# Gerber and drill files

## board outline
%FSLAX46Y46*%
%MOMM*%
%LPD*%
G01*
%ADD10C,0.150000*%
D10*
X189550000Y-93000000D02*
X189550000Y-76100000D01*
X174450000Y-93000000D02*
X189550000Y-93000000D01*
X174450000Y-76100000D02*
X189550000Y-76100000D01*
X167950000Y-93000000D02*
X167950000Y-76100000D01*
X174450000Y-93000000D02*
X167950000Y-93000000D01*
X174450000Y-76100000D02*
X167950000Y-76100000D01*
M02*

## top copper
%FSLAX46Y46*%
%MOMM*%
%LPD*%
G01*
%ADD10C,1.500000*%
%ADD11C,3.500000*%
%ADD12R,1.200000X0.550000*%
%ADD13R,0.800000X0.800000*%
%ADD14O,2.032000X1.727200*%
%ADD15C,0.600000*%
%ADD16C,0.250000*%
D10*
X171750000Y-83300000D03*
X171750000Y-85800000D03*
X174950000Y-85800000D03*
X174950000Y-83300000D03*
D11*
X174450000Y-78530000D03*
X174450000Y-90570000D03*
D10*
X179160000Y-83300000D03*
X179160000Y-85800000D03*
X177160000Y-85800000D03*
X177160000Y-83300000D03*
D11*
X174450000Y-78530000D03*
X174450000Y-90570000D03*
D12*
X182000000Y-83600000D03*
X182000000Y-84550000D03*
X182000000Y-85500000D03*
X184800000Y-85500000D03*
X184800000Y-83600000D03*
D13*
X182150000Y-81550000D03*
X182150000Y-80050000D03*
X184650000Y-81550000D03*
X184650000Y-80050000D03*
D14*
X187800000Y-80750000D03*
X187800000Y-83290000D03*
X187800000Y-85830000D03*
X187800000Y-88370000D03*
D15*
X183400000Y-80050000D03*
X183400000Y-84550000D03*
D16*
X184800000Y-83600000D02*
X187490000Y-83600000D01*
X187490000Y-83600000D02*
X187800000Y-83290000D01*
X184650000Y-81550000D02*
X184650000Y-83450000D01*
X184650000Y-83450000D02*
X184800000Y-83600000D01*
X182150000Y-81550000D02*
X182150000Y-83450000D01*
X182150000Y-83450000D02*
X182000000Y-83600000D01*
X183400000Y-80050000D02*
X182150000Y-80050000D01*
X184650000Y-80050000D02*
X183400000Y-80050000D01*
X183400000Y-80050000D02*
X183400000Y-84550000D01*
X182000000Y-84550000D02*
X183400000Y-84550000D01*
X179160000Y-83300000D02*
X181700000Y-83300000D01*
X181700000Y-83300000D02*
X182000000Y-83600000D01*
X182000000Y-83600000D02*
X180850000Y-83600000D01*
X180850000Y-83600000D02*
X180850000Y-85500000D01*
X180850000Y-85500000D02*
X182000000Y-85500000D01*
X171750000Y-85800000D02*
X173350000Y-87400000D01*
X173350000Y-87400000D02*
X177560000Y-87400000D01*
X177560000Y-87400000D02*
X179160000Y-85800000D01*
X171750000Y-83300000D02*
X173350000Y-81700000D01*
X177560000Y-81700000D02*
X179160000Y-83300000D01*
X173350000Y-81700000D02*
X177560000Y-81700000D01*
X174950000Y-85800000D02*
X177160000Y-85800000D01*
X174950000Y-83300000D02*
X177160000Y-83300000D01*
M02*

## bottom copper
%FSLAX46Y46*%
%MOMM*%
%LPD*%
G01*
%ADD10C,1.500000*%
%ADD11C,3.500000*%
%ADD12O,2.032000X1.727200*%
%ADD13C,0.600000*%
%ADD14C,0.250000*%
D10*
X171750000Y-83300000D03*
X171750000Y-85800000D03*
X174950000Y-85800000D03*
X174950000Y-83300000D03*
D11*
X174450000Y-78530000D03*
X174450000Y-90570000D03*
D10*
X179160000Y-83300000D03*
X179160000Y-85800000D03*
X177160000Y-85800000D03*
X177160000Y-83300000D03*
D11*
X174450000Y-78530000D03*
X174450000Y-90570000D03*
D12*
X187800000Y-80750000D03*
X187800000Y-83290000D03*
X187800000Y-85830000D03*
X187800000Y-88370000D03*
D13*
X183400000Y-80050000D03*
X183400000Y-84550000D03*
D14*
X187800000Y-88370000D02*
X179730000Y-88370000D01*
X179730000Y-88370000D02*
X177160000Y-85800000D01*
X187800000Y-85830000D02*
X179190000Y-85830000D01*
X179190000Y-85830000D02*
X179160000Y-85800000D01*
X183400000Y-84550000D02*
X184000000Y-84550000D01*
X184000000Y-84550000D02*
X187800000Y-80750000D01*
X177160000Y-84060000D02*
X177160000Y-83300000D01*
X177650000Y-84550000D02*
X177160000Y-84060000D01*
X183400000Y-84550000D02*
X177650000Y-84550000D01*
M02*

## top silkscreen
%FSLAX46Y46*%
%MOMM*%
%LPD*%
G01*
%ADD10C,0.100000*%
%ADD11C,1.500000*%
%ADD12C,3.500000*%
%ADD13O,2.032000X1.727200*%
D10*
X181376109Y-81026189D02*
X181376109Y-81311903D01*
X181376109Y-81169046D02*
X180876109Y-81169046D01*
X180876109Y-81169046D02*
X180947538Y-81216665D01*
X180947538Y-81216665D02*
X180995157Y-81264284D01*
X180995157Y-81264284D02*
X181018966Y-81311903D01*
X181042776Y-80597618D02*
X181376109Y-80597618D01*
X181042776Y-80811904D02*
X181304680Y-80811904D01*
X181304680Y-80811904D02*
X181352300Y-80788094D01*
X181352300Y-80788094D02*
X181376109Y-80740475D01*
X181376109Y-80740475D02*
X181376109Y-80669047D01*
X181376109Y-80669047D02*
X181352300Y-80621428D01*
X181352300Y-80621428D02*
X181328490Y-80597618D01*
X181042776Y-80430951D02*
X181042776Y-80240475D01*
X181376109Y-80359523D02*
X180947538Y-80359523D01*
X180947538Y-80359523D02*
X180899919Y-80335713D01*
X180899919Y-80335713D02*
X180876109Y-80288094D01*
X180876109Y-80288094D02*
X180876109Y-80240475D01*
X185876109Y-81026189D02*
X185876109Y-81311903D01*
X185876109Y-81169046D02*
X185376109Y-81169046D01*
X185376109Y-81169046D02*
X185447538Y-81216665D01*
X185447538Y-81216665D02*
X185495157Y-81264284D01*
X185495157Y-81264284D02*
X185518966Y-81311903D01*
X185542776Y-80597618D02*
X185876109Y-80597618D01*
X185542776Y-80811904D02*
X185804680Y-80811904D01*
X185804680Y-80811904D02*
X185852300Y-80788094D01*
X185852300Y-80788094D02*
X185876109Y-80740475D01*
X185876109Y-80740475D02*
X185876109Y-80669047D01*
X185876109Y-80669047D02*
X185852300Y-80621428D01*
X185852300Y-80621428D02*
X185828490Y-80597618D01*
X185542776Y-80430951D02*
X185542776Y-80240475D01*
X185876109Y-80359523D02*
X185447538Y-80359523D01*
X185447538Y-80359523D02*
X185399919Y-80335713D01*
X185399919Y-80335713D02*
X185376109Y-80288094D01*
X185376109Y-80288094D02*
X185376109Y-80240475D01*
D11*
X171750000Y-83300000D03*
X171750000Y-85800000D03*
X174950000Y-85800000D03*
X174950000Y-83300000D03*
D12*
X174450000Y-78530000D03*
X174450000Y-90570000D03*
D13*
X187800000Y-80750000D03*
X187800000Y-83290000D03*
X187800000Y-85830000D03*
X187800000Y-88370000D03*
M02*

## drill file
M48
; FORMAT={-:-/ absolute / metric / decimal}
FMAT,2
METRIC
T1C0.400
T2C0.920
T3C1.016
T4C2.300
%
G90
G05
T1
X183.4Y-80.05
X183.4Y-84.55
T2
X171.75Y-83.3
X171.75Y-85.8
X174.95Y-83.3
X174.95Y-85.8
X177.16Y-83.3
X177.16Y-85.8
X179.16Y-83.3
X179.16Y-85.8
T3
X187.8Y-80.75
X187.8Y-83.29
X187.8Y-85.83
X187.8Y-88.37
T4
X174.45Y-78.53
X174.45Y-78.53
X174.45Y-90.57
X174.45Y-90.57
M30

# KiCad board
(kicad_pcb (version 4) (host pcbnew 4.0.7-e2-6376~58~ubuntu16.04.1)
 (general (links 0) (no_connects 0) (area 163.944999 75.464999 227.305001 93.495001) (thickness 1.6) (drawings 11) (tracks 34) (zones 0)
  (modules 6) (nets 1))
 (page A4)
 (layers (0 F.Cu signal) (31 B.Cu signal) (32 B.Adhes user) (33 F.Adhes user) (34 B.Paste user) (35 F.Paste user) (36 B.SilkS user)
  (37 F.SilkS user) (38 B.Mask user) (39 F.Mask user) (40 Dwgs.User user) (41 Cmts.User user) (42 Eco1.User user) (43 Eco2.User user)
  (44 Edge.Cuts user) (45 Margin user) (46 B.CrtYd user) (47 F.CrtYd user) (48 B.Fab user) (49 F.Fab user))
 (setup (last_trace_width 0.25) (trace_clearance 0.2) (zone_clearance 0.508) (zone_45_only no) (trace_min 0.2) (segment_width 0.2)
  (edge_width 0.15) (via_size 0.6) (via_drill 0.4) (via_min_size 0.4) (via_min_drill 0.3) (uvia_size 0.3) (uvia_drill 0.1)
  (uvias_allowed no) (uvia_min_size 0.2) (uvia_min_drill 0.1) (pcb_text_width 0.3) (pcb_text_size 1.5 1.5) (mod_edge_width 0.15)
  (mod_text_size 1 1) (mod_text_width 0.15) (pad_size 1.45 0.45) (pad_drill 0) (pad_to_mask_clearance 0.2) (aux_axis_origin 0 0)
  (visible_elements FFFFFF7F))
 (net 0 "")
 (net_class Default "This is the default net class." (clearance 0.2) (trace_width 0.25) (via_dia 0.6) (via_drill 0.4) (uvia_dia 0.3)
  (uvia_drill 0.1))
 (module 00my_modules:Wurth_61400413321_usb (layer F.Cu) (at 174.45 84.55 90)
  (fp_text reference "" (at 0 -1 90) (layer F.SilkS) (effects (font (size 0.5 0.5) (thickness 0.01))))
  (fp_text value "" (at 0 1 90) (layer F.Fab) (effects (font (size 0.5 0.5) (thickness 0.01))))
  (pad V thru_hole circle (at 1.25 -2.7 90) (size 1.5 1.5) (drill 0.92) (layers *.Cu *.Mask F.SilkS))
  (pad - thru_hole circle (at -1.25 -2.7 90) (size 1.5 1.5) (drill 0.92) (layers *.Cu *.Mask F.SilkS))
  (pad + thru_hole circle (at -1.25 0.5 90) (size 1.5 1.5) (drill 0.92) (layers *.Cu *.Mask F.SilkS))
  (pad G thru_hole circle (at 1.25 0.5 90) (size 1.5 1.5) (drill 0.92) (layers *.Cu *.Mask F.SilkS))
  (pad X thru_hole circle (at 6.02 0 90) (size 3.5 3.5) (drill 2.3) (layers *.Cu *.Mask F.SilkS))
  (pad X thru_hole circle (at -6.02 0 90) (size 3.5 3.5) (drill 2.3) (layers *.Cu *.Mask F.SilkS)))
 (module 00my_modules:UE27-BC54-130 (layer B.Cu) (at 174.45 84.55 90)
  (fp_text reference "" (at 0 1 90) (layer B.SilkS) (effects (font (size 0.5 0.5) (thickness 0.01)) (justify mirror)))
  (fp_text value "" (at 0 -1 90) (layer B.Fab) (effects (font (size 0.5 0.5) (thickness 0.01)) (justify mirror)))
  (pad V thru_hole circle (at 1.25 4.71 90) (size 1.5 1.5) (drill 0.92) (layers *.Cu *.Mask B.SilkS))
  (pad - thru_hole circle (at -1.25 4.71 90) (size 1.5 1.5) (drill 0.92) (layers *.Cu *.Mask B.SilkS))
  (pad + thru_hole circle (at -1.25 2.71 90) (size 1.5 1.5) (drill 0.92) (layers *.Cu *.Mask B.SilkS))
  (pad G thru_hole circle (at 1.25 2.71 90) (size 1.5 1.5) (drill 0.92) (layers *.Cu *.Mask B.SilkS))
  (pad X thru_hole circle (at 6.02 0 90) (size 3.5 3.5) (drill 2.3) (layers *.Cu *.Mask B.SilkS))
  (pad X thru_hole circle (at -6.02 0 90) (size 3.5 3.5) (drill 2.3) (layers *.Cu *.Mask B.SilkS)))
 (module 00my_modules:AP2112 (layer F.Cu) (at 183.4 84.55)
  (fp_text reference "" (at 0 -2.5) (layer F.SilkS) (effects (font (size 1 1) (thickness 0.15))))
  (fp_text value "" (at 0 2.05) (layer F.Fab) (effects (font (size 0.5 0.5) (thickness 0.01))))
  (pad VIN smd rect (at -1.4 -0.95) (size 1.2 0.55) (layers F.Cu F.Paste F.Mask))
  (pad GND smd rect (at -1.4 0) (size 1.2 0.55) (layers F.Cu F.Paste F.Mask))
  (pad EN smd rect (at -1.4 0.95) (size 1.2 0.55) (layers F.Cu F.Paste F.Mask))
  (pad NC smd rect (at 1.4 0.95) (size 1.2 0.55) (layers F.Cu F.Paste F.Mask))
  (pad VOUT smd rect (at 1.4 -0.95) (size 1.2 0.55) (layers F.Cu F.Paste F.Mask)))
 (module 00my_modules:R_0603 (layer F.Cu) (at 182.15 80.8 90)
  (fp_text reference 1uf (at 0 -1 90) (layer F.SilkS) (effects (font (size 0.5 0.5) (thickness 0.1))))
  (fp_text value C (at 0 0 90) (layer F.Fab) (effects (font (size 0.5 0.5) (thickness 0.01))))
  (pad 1 smd rect (at -0.75 0 90) (size 0.8 0.8) (layers F.Cu F.Paste F.Mask))
  (pad 2 smd rect (at 0.75 0 90) (size 0.8 0.8) (layers F.Cu F.Paste F.Mask)))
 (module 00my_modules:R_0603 (layer F.Cu) (at 184.65 80.8 90)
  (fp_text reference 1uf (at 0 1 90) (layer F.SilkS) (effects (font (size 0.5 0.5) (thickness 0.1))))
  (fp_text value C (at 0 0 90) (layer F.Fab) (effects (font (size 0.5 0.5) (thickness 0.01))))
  (pad 1 smd rect (at -0.75 0 90) (size 0.8 0.8) (layers F.Cu F.Paste F.Mask))
  (pad 2 smd rect (at 0.75 0 90) (size 0.8 0.8) (layers F.Cu F.Paste F.Mask)))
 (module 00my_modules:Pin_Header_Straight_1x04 (layer F.Cu) (at 187.8 80.75)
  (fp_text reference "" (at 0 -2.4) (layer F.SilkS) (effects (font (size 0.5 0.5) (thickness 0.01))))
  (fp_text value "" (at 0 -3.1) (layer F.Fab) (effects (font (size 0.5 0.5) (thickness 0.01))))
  (pad 1 thru_hole oval (at 0 0) (size 2.032 1.7272) (drill 1.016) (layers *.Cu *.Mask F.SilkS))
  (pad 2 thru_hole oval (at 0 2.54) (size 2.032 1.7272) (drill 1.016) (layers *.Cu *.Mask F.SilkS))
  (pad 3 thru_hole oval (at 0 5.08) (size 2.032 1.7272) (drill 1.016) (layers *.Cu *.Mask F.SilkS))
  (pad 4 thru_hole oval (at 0 7.62) (size 2.032 1.7272) (drill 1.016) (layers *.Cu *.Mask F.SilkS)))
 (gr_line (start 189.55 93) (end 189.55 76.1) (angle 90) (layer Edge.Cuts) (width 0.15))
 (gr_line (start 174.45 93) (end 189.55 93) (angle 90) (layer Edge.Cuts) (width 0.15))
 (gr_line (start 174.45 76.1) (end 189.55 76.1) (angle 90) (layer Edge.Cuts) (width 0.15))
 (gr_line (start 167.95 93) (end 167.95 76.1) (angle 90) (layer Edge.Cuts) (width 0.15))
 (gr_line (start 174.45 93) (end 167.95 93) (angle 90) (layer Edge.Cuts) (width 0.15))
 (gr_line (start 174.45 76.1) (end 167.95 76.1) (angle 90) (layer Edge.Cuts) (width 0.15))
 (segment (start 187.8 88.37) (end 179.73 88.37) (width 0.25) (layer B.Cu) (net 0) (status 400000))
 (segment (start 179.73 88.37) (end 177.16 85.8) (width 0.25) (layer B.Cu) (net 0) (status 800000))
 (segment (start 187.8 85.83) (end 179.19 85.83) (width 0.25) (layer B.Cu) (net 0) (status C00000))
 (segment (start 179.19 85.83) (end 179.16 85.8) (width 0.25) (layer B.Cu) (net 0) (status C00000))
 (segment (start 184.8 83.6) (end 187.49 83.6) (width 0.25) (layer F.Cu) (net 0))
 (segment (start 187.49 83.6) (end 187.8 83.29) (width 0.25) (layer F.Cu) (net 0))
 (segment (start 183.4 84.55) (end 184 84.55) (width 0.25) (layer B.Cu) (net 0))
 (segment (start 184 84.55) (end 187.8 80.75) (width 0.25) (layer B.Cu) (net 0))
 (segment (start 184.65 81.55) (end 184.65 83.45) (width 0.25) (layer F.Cu) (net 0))
 (segment (start 184.65 83.45) (end 184.8 83.6) (width 0.25) (layer F.Cu) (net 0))
 (segment (start 182.15 81.55) (end 182.15 83.45) (width 0.25) (layer F.Cu) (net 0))
 (segment (start 182.15 83.45) (end 182 83.6) (width 0.25) (layer F.Cu) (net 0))
 (segment (start 183.4 80.05) (end 182.15 80.05) (width 0.25) (layer F.Cu) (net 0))
 (via (at 183.4 80.05) (size 0.6) (drill 0.4) (layers F.Cu B.Cu) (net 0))
 (segment (start 184.65 80.05) (end 183.4 80.05) (width 0.25) (layer F.Cu) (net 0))
 (segment (start 183.4 80.05) (end 183.4 84.55) (width 0.25) (layer F.Cu) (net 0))
 (segment (start 182 84.55) (end 183.4 84.55) (width 0.25) (layer F.Cu) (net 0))
 (segment (start 177.16 84.06) (end 177.16 83.3) (width 0.25) (layer B.Cu) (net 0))
 (segment (start 177.65 84.55) (end 177.16 84.06) (width 0.25) (layer B.Cu) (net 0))
 (segment (start 183.4 84.55) (end 177.65 84.55) (width 0.25) (layer B.Cu) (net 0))
 (via (at 183.4 84.55) (size 0.6) (drill 0.4) (layers F.Cu B.Cu) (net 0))
 (segment (start 179.16 83.3) (end 181.7 83.3) (width 0.25) (layer F.Cu) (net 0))
 (segment (start 181.7 83.3) (end 182 83.6) (width 0.25) (layer F.Cu) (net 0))
 (segment (start 182 83.6) (end 180.85 83.6) (width 0.25) (layer F.Cu) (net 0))
 (segment (start 180.85 83.6) (end 180.85 85.5) (width 0.25) (layer F.Cu) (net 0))
 (segment (start 180.85 85.5) (end 182 85.5) (width 0.25) (layer F.Cu) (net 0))
 (segment (start 171.75 85.8) (end 173.35 87.4) (width 0.25) (layer F.Cu) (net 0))
 (segment (start 173.35 87.4) (end 177.56 87.4) (width 0.25) (layer F.Cu) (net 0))
 (segment (start 177.56 87.4) (end 179.16 85.8) (width 0.25) (layer F.Cu) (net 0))
 (segment (start 171.75 83.3) (end 173.35 81.7) (width 0.25) (layer F.Cu) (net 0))
 (segment (start 177.56 81.7) (end 179.16 83.3) (width 0.25) (layer F.Cu) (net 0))
 (segment (start 173.35 81.7) (end 177.56 81.7) (width 0.25) (layer F.Cu) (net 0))
 (segment (start 174.95 85.8) (end 177.16 85.8) (width 0.25) (layer F.Cu) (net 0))
 (segment (start 174.95 83.3) (end 177.16 83.3) (width 0.25) (layer F.Cu) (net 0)))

